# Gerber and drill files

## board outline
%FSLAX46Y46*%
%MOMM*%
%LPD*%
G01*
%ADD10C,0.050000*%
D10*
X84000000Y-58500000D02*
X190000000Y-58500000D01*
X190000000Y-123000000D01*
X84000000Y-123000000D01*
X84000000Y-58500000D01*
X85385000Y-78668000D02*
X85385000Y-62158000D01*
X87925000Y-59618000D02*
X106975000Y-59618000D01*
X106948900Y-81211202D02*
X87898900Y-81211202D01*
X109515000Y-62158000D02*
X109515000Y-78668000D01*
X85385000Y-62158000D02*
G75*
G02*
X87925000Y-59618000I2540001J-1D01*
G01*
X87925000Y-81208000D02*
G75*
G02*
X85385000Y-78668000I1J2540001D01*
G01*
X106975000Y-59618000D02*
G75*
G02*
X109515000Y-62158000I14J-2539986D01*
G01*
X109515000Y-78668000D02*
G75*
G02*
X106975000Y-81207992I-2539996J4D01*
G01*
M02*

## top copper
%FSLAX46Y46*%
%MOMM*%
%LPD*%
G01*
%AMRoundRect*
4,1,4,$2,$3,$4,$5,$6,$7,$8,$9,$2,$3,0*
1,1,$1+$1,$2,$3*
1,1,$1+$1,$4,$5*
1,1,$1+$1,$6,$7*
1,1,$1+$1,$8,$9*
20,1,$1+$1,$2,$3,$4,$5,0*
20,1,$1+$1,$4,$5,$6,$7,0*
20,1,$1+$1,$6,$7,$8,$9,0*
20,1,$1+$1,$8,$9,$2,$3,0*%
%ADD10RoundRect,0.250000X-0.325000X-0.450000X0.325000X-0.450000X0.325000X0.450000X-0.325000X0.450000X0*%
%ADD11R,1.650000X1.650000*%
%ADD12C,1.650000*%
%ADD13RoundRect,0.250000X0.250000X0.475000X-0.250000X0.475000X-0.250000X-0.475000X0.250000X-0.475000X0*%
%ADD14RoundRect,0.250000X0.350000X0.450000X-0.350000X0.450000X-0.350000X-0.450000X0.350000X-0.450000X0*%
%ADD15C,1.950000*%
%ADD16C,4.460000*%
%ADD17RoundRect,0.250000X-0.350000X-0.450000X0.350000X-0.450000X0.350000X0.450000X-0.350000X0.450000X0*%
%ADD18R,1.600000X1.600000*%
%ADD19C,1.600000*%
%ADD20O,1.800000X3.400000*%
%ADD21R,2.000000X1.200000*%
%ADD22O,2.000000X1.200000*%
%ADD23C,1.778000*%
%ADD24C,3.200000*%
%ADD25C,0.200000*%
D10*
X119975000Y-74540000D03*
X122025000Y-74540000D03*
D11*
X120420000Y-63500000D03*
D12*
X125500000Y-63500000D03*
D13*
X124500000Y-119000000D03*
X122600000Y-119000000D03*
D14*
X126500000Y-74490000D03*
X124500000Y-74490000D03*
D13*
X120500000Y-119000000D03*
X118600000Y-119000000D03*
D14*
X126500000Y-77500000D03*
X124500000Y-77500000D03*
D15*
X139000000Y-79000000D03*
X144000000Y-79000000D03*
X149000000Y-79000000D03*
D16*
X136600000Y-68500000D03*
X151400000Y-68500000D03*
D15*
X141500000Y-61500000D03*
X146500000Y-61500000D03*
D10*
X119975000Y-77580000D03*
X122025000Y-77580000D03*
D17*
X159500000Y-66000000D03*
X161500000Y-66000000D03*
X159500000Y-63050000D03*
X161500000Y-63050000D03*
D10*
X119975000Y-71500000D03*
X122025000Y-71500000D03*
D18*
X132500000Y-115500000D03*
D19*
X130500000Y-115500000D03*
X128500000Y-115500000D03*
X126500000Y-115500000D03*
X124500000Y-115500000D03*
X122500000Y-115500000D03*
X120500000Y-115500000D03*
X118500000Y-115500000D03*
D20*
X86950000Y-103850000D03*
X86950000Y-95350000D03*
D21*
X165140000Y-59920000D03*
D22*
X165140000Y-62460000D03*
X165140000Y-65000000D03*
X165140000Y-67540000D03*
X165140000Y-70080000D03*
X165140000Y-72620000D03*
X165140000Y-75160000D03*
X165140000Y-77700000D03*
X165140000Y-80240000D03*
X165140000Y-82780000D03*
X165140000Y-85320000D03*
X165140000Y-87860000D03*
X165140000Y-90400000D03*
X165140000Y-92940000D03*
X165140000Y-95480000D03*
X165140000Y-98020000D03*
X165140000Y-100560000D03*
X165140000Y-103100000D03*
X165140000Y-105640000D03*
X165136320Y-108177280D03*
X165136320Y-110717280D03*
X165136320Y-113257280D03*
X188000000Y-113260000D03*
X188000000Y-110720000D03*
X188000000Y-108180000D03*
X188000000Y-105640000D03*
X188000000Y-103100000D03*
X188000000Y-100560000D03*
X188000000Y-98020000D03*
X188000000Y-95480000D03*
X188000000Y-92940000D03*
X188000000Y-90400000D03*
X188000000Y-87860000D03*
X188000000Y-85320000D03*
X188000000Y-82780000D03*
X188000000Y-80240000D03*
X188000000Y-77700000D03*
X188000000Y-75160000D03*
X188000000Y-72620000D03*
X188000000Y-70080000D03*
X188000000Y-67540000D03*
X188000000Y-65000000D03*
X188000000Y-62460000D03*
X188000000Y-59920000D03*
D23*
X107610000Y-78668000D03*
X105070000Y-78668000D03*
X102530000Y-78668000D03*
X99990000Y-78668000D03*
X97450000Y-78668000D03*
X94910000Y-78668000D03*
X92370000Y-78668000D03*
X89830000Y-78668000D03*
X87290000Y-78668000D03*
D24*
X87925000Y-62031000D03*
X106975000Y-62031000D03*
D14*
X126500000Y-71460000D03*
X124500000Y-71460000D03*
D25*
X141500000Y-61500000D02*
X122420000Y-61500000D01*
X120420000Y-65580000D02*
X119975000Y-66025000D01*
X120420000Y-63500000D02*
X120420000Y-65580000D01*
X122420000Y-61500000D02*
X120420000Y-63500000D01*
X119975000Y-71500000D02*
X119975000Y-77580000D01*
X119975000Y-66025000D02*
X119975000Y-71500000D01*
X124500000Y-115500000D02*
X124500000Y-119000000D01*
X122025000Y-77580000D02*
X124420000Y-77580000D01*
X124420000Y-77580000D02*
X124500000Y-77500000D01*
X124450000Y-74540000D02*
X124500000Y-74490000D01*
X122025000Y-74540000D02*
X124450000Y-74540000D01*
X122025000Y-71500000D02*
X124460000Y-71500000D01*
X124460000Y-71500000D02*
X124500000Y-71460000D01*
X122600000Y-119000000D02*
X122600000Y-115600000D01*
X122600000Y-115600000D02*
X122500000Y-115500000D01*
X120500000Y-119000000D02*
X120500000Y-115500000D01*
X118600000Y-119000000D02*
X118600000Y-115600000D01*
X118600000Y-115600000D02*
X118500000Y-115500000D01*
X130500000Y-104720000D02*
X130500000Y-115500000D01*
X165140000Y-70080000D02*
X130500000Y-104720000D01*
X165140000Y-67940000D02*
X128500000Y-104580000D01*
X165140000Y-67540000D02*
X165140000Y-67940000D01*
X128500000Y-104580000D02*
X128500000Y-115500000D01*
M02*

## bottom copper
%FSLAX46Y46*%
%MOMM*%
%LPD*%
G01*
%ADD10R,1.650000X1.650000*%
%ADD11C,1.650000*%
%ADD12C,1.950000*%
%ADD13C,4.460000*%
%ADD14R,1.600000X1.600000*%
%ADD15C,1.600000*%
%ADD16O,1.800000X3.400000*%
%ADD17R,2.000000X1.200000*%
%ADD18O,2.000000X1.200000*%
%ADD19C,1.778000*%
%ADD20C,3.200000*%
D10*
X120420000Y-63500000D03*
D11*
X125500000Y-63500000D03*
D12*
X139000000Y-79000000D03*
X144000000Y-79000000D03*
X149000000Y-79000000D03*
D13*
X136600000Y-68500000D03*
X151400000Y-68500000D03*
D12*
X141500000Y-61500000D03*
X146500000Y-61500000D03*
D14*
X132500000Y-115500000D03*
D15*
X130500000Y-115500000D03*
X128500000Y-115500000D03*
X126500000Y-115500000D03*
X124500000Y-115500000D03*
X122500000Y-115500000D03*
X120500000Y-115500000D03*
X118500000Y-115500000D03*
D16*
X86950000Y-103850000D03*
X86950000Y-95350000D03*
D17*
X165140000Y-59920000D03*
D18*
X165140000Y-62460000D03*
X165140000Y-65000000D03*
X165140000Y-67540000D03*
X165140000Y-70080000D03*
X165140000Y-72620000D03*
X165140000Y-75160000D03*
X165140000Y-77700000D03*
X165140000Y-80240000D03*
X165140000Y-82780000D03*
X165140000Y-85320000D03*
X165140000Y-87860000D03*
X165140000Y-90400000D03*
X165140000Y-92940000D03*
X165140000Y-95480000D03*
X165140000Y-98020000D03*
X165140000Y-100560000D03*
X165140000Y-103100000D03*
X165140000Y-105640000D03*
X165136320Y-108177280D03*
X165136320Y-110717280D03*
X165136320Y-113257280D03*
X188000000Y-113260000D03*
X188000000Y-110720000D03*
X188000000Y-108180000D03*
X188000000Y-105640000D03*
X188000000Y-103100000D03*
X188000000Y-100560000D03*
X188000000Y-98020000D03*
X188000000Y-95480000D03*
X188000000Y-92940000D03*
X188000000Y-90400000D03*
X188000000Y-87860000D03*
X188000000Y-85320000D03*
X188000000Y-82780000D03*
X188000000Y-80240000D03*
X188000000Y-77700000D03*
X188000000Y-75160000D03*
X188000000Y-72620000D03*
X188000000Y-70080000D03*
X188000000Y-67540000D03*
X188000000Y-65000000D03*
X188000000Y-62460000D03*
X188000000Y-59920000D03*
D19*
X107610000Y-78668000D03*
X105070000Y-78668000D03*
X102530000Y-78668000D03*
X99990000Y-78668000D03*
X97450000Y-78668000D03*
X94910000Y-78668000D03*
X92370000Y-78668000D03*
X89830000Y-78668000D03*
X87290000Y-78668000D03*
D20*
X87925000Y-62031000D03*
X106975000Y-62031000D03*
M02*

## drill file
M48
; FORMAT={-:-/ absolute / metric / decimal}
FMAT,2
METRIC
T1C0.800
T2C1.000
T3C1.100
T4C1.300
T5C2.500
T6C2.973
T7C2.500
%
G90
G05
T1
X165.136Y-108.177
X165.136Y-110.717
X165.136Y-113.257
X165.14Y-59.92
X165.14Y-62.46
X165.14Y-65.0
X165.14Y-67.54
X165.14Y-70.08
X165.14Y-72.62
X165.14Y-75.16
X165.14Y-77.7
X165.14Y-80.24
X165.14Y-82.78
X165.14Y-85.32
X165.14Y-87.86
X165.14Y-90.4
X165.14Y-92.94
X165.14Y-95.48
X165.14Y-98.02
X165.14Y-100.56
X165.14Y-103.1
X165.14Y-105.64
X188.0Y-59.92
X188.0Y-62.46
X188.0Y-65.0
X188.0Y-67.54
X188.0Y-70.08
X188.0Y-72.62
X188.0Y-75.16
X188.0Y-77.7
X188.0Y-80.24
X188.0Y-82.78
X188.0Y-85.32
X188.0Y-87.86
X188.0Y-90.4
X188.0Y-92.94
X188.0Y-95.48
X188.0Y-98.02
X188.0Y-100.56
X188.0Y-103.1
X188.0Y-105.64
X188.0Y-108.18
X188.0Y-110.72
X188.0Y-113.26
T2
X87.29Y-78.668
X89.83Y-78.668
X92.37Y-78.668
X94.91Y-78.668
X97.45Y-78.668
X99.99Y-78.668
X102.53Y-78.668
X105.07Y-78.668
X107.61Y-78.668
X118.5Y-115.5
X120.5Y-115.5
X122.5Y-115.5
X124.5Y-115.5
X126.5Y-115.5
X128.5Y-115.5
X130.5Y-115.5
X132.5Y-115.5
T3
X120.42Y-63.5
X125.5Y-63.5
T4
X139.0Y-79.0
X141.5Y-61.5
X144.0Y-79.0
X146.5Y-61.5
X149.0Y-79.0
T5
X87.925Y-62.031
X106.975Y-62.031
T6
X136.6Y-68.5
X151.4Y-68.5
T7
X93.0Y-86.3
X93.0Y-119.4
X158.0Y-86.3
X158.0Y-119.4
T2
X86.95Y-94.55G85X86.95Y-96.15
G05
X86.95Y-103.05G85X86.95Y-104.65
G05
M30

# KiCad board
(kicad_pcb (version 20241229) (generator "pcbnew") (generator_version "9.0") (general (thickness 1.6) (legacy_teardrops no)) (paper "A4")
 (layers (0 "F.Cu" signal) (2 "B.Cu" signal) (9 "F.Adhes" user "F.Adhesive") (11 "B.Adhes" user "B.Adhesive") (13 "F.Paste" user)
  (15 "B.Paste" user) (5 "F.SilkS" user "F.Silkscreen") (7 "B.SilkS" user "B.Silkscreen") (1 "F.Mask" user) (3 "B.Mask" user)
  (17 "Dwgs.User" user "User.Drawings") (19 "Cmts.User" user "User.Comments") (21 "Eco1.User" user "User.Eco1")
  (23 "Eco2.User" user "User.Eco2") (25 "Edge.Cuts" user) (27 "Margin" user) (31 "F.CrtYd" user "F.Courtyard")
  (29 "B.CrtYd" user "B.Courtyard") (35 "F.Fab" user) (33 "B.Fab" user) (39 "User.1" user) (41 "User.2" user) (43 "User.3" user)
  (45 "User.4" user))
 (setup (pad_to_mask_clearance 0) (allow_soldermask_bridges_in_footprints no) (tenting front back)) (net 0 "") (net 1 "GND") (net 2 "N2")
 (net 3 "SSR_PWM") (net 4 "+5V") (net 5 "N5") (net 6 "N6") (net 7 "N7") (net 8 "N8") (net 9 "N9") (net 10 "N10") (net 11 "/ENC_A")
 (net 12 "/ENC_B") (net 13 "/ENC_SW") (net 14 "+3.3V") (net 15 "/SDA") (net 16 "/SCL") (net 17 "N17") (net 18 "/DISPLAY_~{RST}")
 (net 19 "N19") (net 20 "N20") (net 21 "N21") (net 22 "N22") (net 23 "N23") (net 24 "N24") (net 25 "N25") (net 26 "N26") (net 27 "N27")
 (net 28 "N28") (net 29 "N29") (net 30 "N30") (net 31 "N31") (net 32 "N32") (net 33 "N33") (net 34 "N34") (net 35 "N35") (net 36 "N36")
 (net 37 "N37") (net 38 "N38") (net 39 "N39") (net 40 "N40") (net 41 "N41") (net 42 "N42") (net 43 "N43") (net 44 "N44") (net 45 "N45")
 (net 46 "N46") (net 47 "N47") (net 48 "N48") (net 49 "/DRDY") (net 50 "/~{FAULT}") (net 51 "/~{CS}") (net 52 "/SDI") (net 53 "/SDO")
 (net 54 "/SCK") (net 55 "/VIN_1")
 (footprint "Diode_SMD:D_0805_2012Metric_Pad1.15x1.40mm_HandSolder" (layer "F.Cu") (at 121 74.54)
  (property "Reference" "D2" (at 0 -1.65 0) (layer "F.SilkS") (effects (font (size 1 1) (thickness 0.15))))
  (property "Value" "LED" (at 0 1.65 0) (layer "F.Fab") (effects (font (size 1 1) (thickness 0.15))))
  (pad "1" smd roundrect (at -1.025 0) (size 1.15 1.4) (layers "F.Cu" "F.Mask" "F.Paste") (roundrect_rratio 0.217391) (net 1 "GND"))
  (pad "2" smd roundrect (at 1.025 0) (size 1.15 1.4) (layers "F.Cu" "F.Mask" "F.Paste") (roundrect_rratio 0.217391) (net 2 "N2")))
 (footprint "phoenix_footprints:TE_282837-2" (layer "F.Cu") (at 122.96 63.5)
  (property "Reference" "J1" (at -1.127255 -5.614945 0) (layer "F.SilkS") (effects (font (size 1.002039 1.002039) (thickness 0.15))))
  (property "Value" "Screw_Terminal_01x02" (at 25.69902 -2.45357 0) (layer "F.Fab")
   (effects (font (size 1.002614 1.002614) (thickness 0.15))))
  (pad "1" thru_hole rect (at -2.54 0) (size 1.65 1.65) (drill 1.1) (layers "*.Cu" "*.Mask") (remove_unused_layers no) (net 1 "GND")
   (solder_mask_margin 0.102))
  (pad "2" thru_hole circle (at 2.54 0) (size 1.65 1.65) (drill 1.1) (layers "*.Cu" "*.Mask") (remove_unused_layers no) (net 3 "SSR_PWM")
   (solder_mask_margin 0.102)))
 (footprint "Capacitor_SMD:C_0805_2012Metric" (layer "F.Cu") (at 123.55 119 180)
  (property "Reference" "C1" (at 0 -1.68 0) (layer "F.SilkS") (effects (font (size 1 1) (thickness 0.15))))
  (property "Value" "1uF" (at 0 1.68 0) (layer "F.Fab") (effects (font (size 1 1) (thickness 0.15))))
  (pad "1" smd roundrect (at -0.95 0 180) (size 1 1.45) (layers "F.Cu" "F.Mask" "F.Paste") (roundrect_rratio 0.25) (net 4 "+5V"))
  (pad "2" smd roundrect (at 0.95 0 180) (size 1 1.45) (layers "F.Cu" "F.Mask" "F.Paste") (roundrect_rratio 0.25) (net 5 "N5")))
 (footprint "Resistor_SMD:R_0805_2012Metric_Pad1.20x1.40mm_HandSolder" (layer "F.Cu") (at 125.5 74.49 180)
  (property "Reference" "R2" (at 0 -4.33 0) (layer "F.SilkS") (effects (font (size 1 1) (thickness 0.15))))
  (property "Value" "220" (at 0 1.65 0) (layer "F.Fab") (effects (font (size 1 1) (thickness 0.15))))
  (pad "1" smd roundrect (at -1 0 180) (size 1.2 1.4) (layers "F.Cu" "F.Mask" "F.Paste") (roundrect_rratio 0.208333) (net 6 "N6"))
  (pad "2" smd roundrect (at 1 0 180) (size 1.2 1.4) (layers "F.Cu" "F.Mask" "F.Paste") (roundrect_rratio 0.208333) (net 2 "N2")))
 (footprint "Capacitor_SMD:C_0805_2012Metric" (layer "F.Cu") (at 119.55 119 180)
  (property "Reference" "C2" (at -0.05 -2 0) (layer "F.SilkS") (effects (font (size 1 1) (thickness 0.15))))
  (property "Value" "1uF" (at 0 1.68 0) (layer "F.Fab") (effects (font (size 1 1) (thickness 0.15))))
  (pad "1" smd roundrect (at -0.95 0 180) (size 1 1.45) (layers "F.Cu" "F.Mask" "F.Paste") (roundrect_rratio 0.25) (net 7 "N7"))
  (pad "2" smd roundrect (at 0.95 0 180) (size 1 1.45) (layers "F.Cu" "F.Mask" "F.Paste") (roundrect_rratio 0.25) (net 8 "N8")))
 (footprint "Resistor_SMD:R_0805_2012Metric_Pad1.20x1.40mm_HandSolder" (layer "F.Cu") (at 125.5 77.5 180)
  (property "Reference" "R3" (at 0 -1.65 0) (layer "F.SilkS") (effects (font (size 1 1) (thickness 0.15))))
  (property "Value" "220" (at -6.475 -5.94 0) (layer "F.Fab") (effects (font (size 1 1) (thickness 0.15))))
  (pad "1" smd roundrect (at -1 0 180) (size 1.2 1.4) (layers "F.Cu" "F.Mask" "F.Paste") (roundrect_rratio 0.208333) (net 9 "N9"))
  (pad "2" smd roundrect (at 1 0 180) (size 1.2 1.4) (layers "F.Cu" "F.Mask" "F.Paste") (roundrect_rratio 0.208333) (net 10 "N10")))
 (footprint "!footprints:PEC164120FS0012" (layer "F.Cu") (at 139 79)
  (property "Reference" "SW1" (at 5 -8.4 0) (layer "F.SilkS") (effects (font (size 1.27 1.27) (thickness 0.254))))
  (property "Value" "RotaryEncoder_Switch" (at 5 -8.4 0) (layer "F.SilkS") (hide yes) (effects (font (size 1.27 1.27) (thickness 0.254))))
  (pad "A" thru_hole circle (at 0 0) (size 1.95 1.95) (drill 1.3) (layers "*.Cu" "*.Mask") (remove_unused_layers no) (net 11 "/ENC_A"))
  (pad "B" thru_hole circle (at 5 0) (size 1.95 1.95) (drill 1.3) (layers "*.Cu" "*.Mask") (remove_unused_layers no) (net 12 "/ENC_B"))
  (pad "C" thru_hole circle (at 10 0) (size 1.95 1.95) (drill 1.3) (layers "*.Cu" "*.Mask") (remove_unused_layers no) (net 1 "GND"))
  (pad "MH1" thru_hole circle (at -2.4 -10.5) (size 4.46 4.46) (drill 2.9732) (layers "*.Cu" "*.Mask") (remove_unused_layers no))
  (pad "MH2" thru_hole circle (at 12.4 -10.5) (size 4.46 4.46) (drill 2.9732) (layers "*.Cu" "*.Mask") (remove_unused_layers no))
  (pad "S1" thru_hole circle (at 2.5 -17.5) (size 1.95 1.95) (drill 1.3) (layers "*.Cu" "*.Mask") (remove_unused_layers no) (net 1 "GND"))
  (pad "S2" thru_hole circle (at 7.5 -17.5) (size 1.95 1.95) (drill 1.3) (layers "*.Cu" "*.Mask") (remove_unused_layers no)
   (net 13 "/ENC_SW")))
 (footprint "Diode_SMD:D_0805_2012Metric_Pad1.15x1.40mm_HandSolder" (layer "F.Cu") (at 121 77.58)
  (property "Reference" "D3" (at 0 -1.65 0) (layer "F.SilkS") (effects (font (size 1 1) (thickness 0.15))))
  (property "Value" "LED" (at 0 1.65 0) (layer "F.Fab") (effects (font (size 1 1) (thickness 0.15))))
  (pad "1" smd roundrect (at -1.025 0) (size 1.15 1.4) (layers "F.Cu" "F.Mask" "F.Paste") (roundrect_rratio 0.217391) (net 1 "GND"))
  (pad "2" smd roundrect (at 1.025 0) (size 1.15 1.4) (layers "F.Cu" "F.Mask" "F.Paste") (roundrect_rratio 0.217391) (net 10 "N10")))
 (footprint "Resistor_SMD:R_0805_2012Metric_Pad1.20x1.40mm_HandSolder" (layer "F.Cu") (at 160.5 66)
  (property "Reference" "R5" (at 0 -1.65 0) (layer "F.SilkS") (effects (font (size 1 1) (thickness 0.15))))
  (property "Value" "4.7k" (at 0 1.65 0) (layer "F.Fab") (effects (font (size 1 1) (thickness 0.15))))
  (pad "1" smd roundrect (at -1 0) (size 1.2 1.4) (layers "F.Cu" "F.Mask" "F.Paste") (roundrect_rratio 0.208333) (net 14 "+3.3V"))
  (pad "2" smd roundrect (at 1 0) (size 1.2 1.4) (layers "F.Cu" "F.Mask" "F.Paste") (roundrect_rratio 0.208333) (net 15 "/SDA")))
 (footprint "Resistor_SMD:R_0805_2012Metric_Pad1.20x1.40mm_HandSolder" (layer "F.Cu") (at 160.5 63.05)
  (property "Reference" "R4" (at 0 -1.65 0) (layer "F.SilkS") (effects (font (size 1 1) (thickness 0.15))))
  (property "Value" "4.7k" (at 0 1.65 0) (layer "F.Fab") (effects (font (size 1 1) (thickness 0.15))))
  (pad "1" smd roundrect (at -1 0) (size 1.2 1.4) (layers "F.Cu" "F.Mask" "F.Paste") (roundrect_rratio 0.208333) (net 14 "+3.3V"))
  (pad "2" smd roundrect (at 1 0) (size 1.2 1.4) (layers "F.Cu" "F.Mask" "F.Paste") (roundrect_rratio 0.208333) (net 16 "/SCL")))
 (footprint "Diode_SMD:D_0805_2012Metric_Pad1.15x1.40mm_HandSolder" (layer "F.Cu") (at 121 71.5)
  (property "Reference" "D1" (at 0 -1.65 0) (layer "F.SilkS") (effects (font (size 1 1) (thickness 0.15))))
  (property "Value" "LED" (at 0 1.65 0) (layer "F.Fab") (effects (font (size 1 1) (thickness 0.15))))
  (pad "1" smd roundrect (at -1.025 0) (size 1.15 1.4) (layers "F.Cu" "F.Mask" "F.Paste") (roundrect_rratio 0.217391) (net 1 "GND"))
  (pad "2" smd roundrect (at 1.025 0) (size 1.15 1.4) (layers "F.Cu" "F.Mask" "F.Paste") (roundrect_rratio 0.217391) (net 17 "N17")))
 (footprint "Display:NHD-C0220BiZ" (layer "F.Cu") (at 125.5 99.6)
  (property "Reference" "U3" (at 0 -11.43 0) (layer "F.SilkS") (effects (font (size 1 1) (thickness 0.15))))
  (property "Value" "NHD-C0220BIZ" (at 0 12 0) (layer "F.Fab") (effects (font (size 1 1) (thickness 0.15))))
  (pad "" np_thru_hole circle (at -32.5 -13.3) (size 2.5 2.5) (drill 2.5) (layers "*.Cu" "*.Mask"))
  (pad "" np_thru_hole circle (at -32.5 19.8) (size 2.5 2.5) (drill 2.5) (layers "*.Cu" "*.Mask"))
  (pad "" np_thru_hole circle (at 32.5 -13.3) (size 2.5 2.5) (drill 2.5) (layers "*.Cu" "*.Mask"))
  (pad "" np_thru_hole circle (at 32.5 19.8) (size 2.5 2.5) (drill 2.5) (layers "*.Cu" "*.Mask"))
  (pad "1" thru_hole rect (at 7 15.9) (size 1.6 1.6) (drill 1) (layers "*.Cu" "*.Mask") (remove_unused_layers no) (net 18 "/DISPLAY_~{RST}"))
  (pad "2" thru_hole circle (at 5 15.9) (size 1.6 1.6) (drill 1) (layers "*.Cu" "*.Mask") (remove_unused_layers no) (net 16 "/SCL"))
  (pad "3" thru_hole circle (at 3 15.9) (size 1.6 1.6) (drill 1) (layers "*.Cu" "*.Mask") (remove_unused_layers no) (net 15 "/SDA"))
  (pad "4" thru_hole circle (at 1 15.9) (size 1.6 1.6) (drill 1) (layers "*.Cu" "*.Mask") (remove_unused_layers no) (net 1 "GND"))
  (pad "5" thru_hole circle (at -1 15.9) (size 1.6 1.6) (drill 1) (layers "*.Cu" "*.Mask") (remove_unused_layers no) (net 4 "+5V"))
  (pad "6" thru_hole circle (at -3 15.9) (size 1.6 1.6) (drill 1) (layers "*.Cu" "*.Mask") (remove_unused_layers no) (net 5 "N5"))
  (pad "7" thru_hole circle (at -5 15.9) (size 1.6 1.6) (drill 1) (layers "*.Cu" "*.Mask") (remove_unused_layers no) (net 7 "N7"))
  (pad "8" thru_hole circle (at -7 15.9) (size 1.6 1.6) (drill 1) (layers "*.Cu" "*.Mask") (remove_unused_layers no) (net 8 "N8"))
  (pad "9" thru_hole oval (at -38.55 4.25) (size 1.8 3.4) (drill oval 1 2.6) (layers "*.Cu" "*.Mask") (remove_unused_layers no)
   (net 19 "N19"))
  (pad "10" thru_hole oval (at -38.55 -4.25) (size 1.8 3.4) (drill oval 1 2.6) (layers "*.Cu" "*.Mask") (remove_unused_layers no)
   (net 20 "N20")))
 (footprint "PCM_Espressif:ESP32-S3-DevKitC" (layer "F.Cu") (at 165.14 59.92)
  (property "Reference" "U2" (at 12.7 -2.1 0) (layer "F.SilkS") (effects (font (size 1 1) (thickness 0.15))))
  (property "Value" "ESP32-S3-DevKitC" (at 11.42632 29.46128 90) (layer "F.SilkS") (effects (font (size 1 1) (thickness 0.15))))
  (pad "1" thru_hole rect (at 0 0 270) (size 1.2 2) (drill 0.8) (layers "*.Cu" "*.Mask") (remove_unused_layers no) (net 14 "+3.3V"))
  (pad "2" thru_hole oval (at 0 2.54 270) (size 1.2 2) (drill 0.8) (layers "*.Cu" "*.Mask") (remove_unused_layers no) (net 14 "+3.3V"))
  (pad "3" thru_hole oval (at 0 5.08 270) (size 1.2 2) (drill 0.8) (layers "*.Cu" "*.Mask") (remove_unused_layers no) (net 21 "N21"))
  (pad "4" thru_hole oval (at 0 7.62 270) (size 1.2 2) (drill 0.8) (layers "*.Cu" "*.Mask") (remove_unused_layers no) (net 15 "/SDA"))
  (pad "5" thru_hole oval (at 0 10.16 270) (size 1.2 2) (drill 0.8) (layers "*.Cu" "*.Mask") (remove_unused_layers no) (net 16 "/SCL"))
  (pad "6" thru_hole oval (at 0 12.7 270) (size 1.2 2) (drill 0.8) (layers "*.Cu" "*.Mask") (remove_unused_layers no) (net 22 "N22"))
  (pad "7" thru_hole oval (at 0 15.24 270) (size 1.2 2) (drill 0.8) (layers "*.Cu" "*.Mask") (remove_unused_layers no) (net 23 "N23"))
  (pad "8" thru_hole oval (at 0 17.78 270) (size 1.2 2) (drill 0.8) (layers "*.Cu" "*.Mask") (remove_unused_layers no) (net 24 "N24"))
  (pad "9" thru_hole oval (at 0 20.32 270) (size 1.2 2) (drill 0.8) (layers "*.Cu" "*.Mask") (remove_unused_layers no) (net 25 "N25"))
  (pad "10" thru_hole oval (at 0 22.86 270) (size 1.2 2) (drill 0.8) (layers "*.Cu" "*.Mask") (remove_unused_layers no) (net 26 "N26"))
  (pad "11" thru_hole oval (at 0 25.4 270) (size 1.2 2) (drill 0.8) (layers "*.Cu" "*.Mask") (remove_unused_layers no) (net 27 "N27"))
  (pad "12" thru_hole oval (at 0 27.94 270) (size 1.2 2) (drill 0.8) (layers "*.Cu" "*.Mask") (remove_unused_layers no) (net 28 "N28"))
  (pad "13" thru_hole oval (at 0 30.48 270) (size 1.2 2) (drill 0.8) (layers "*.Cu" "*.Mask") (remove_unused_layers no) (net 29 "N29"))
  (pad "14" thru_hole oval (at 0 33.02 270) (size 1.2 2) (drill 0.8) (layers "*.Cu" "*.Mask") (remove_unused_layers no) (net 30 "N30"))
  (pad "15" thru_hole oval (at 0 35.56 270) (size 1.2 2) (drill 0.8) (layers "*.Cu" "*.Mask") (remove_unused_layers no) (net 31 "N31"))
  (pad "16" thru_hole oval (at 0 38.1 270) (size 1.2 2) (drill 0.8) (layers "*.Cu" "*.Mask") (remove_unused_layers no) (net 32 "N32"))
  (pad "17" thru_hole oval (at 0 40.64 270) (size 1.2 2) (drill 0.8) (layers "*.Cu" "*.Mask") (remove_unused_layers no) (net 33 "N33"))
  (pad "18" thru_hole oval (at 0 43.18 270) (size 1.2 2) (drill 0.8) (layers "*.Cu" "*.Mask") (remove_unused_layers no) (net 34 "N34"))
  (pad "19" thru_hole oval (at 0 45.72 270) (size 1.2 2) (drill 0.8) (layers "*.Cu" "*.Mask") (remove_unused_layers no) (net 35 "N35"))
  (pad "20" thru_hole oval (at -0.00368 48.25728 270) (size 1.2 2) (drill 0.8) (layers "*.Cu" "*.Mask") (remove_unused_layers no)
   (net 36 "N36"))
  (pad "21" thru_hole oval (at -0.00368 50.79728 270) (size 1.2 2) (drill 0.8) (layers "*.Cu" "*.Mask") (remove_unused_layers no)
   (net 4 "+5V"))
  (pad "22" thru_hole oval (at -0.00368 53.33728 270) (size 1.2 2) (drill 0.8) (layers "*.Cu" "*.Mask") (remove_unused_layers no)
   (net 1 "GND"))
  (pad "23" thru_hole oval (at 22.86 53.34 270) (size 1.2 2) (drill 0.8) (layers "*.Cu" "*.Mask") (remove_unused_layers no) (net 1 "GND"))
  (pad "24" thru_hole oval (at 22.86 50.8 270) (size 1.2 2) (drill 0.8) (layers "*.Cu" "*.Mask") (remove_unused_layers no) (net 1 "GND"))
  (pad "25" thru_hole oval (at 22.86 48.26 270) (size 1.2 2) (drill 0.8) (layers "*.Cu" "*.Mask") (remove_unused_layers no) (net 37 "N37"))
  (pad "26" thru_hole oval (at 22.86 45.72 270) (size 1.2 2) (drill 0.8) (layers "*.Cu" "*.Mask") (remove_unused_layers no) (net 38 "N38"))
  (pad "27" thru_hole oval (at 22.86 43.18 270) (size 1.2 2) (drill 0.8) (layers "*.Cu" "*.Mask") (remove_unused_layers no)
   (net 3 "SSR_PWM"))
  (pad "28" thru_hole oval (at 22.86 40.64 270) (size 1.2 2) (drill 0.8) (layers "*.Cu" "*.Mask") (remove_unused_layers no) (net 6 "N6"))
  (pad "29" thru_hole oval (at 22.86 38.1 270) (size 1.2 2) (drill 0.8) (layers "*.Cu" "*.Mask") (remove_unused_layers no) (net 9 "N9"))
  (pad "30" thru_hole oval (at 22.86 35.56 270) (size 1.2 2) (drill 0.8) (layers "*.Cu" "*.Mask") (remove_unused_layers no) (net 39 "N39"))
  (pad "31" thru_hole oval (at 22.86 33.02 270) (size 1.2 2) (drill 0.8) (layers "*.Cu" "*.Mask") (remove_unused_layers no) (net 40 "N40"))
  (pad "32" thru_hole oval (at 22.86 30.48 270) (size 1.2 2) (drill 0.8) (layers "*.Cu" "*.Mask") (remove_unused_layers no)
   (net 18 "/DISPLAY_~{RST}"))
  (pad "33" thru_hole oval (at 22.86 27.94 270) (size 1.2 2) (drill 0.8) (layers "*.Cu" "*.Mask") (remove_unused_layers no)
   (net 11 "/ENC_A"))
  (pad "34" thru_hole oval (at 22.86 25.4 270) (size 1.2 2) (drill 0.8) (layers "*.Cu" "*.Mask") (remove_unused_layers no) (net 12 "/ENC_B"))
  (pad "35" thru_hole oval (at 22.86 22.86 270) (size 1.2 2) (drill 0.8) (layers "*.Cu" "*.Mask") (remove_unused_layers no)
   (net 13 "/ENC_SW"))
  (pad "36" thru_hole oval (at 22.86 20.32 270) (size 1.2 2) (drill 0.8) (layers "*.Cu" "*.Mask") (remove_unused_layers no) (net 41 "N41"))
  (pad "37" thru_hole oval (at 22.86 17.78 270) (size 1.2 2) (drill 0.8) (layers "*.Cu" "*.Mask") (remove_unused_layers no) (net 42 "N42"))
  (pad "38" thru_hole oval (at 22.86 15.24 270) (size 1.2 2) (drill 0.8) (layers "*.Cu" "*.Mask") (remove_unused_layers no) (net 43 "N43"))
  (pad "39" thru_hole oval (at 22.86 12.7 270) (size 1.2 2) (drill 0.8) (layers "*.Cu" "*.Mask") (remove_unused_layers no) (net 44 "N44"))
  (pad "40" thru_hole oval (at 22.86 10.16 270) (size 1.2 2) (drill 0.8) (layers "*.Cu" "*.Mask") (remove_unused_layers no) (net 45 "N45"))
  (pad "41" thru_hole oval (at 22.86 7.62 270) (size 1.2 2) (drill 0.8) (layers "*.Cu" "*.Mask") (remove_unused_layers no) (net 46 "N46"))
  (pad "42" thru_hole oval (at 22.86 5.08 270) (size 1.2 2) (drill 0.8) (layers "*.Cu" "*.Mask") (remove_unused_layers no) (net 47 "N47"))
  (pad "43" thru_hole oval (at 22.86 2.54 270) (size 1.2 2) (drill 0.8) (layers "*.Cu" "*.Mask") (remove_unused_layers no) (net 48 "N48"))
  (pad "44" thru_hole oval (at 22.86 0 270) (size 1.2 2) (drill 0.8) (layers "*.Cu" "*.Mask") (remove_unused_layers no) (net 1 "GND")))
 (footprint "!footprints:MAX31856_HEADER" (layer "F.Cu") (at 87.936314 62.019686)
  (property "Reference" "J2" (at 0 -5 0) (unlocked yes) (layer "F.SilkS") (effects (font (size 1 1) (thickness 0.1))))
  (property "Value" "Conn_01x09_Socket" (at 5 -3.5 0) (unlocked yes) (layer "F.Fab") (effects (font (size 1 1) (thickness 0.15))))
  (fp_line (start -2.551314 16.648314) (end -2.551314 0.138314) (stroke (width 0.05) (type solid)) (layer "Edge.Cuts"))
  (fp_line (start -0.011314 -2.401686) (end 19.038686 -2.401686) (stroke (width 0.05) (type solid)) (layer "Edge.Cuts"))
  (fp_line (start 19.012586 19.191516) (end -0.037414 19.191516) (stroke (width 0.05) (type solid)) (layer "Edge.Cuts"))
  (fp_line (start 21.578686 0.138314) (end 21.578686 16.648314) (stroke (width 0.05) (type solid)) (layer "Edge.Cuts"))
  (fp_arc (start -2.551314 0.138314) (mid -1.807365 -1.657737) (end -0.011314 -2.401686) (stroke (width 0.05) (type solid))
   (layer "Edge.Cuts"))
  (fp_arc (start -0.011314 19.188314) (mid -1.807365 18.444365) (end -2.551314 16.648314) (stroke (width 0.05) (type solid))
   (layer "Edge.Cuts"))
  (fp_arc (start 19.038686 -2.401686) (mid 20.834737 -1.657737) (end 21.578686 0.138314) (stroke (width 0.05) (type solid))
   (layer "Edge.Cuts"))
  (fp_arc (start 21.578686 16.648314) (mid 20.834737 18.444365) (end 19.038686 19.188314) (stroke (width 0.05) (type solid))
   (layer "Edge.Cuts"))
  (pad "1" thru_hole circle (at 19.673686 16.648314 270) (size 1.778 1.778) (drill 1) (layers "*.Cu" "*.Mask") (remove_unused_layers no)
   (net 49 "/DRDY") (solder_mask_margin 0.0508) (thermal_bridge_angle 0))
  (pad "2" thru_hole circle (at 17.133686 16.648314 270) (size 1.778 1.778) (drill 1) (layers "*.Cu" "*.Mask") (remove_unused_layers no)
   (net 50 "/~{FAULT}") (solder_mask_margin 0.0508) (thermal_bridge_angle 0))
  (pad "3" thru_hole circle (at 14.593686 16.648314 270) (size 1.778 1.778) (drill 1) (layers "*.Cu" "*.Mask") (remove_unused_layers no)
   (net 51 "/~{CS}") (solder_mask_margin 0.0508) (thermal_bridge_angle 0))
  (pad "4" thru_hole circle (at 12.053686 16.648314 270) (size 1.778 1.778) (drill 1) (layers "*.Cu" "*.Mask") (remove_unused_layers no)
   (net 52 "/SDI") (solder_mask_margin 0.0508) (thermal_bridge_angle 0))
  (pad "5" thru_hole circle (at 9.513686 16.648314 270) (size 1.778 1.778) (drill 1) (layers "*.Cu" "*.Mask") (remove_unused_layers no)
   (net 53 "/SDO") (solder_mask_margin 0.0508) (thermal_bridge_angle 0))
  (pad "6" thru_hole circle (at 6.973686 16.648314 270) (size 1.778 1.778) (drill 1) (layers "*.Cu" "*.Mask") (remove_unused_layers no)
   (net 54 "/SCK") (solder_mask_margin 0.0508) (thermal_bridge_angle 0))
  (pad "7" thru_hole circle (at 4.433686 16.648314 270) (size 1.778 1.778) (drill 1) (layers "*.Cu" "*.Mask") (remove_unused_layers no)
   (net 1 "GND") (solder_mask_margin 0.0508) (thermal_bridge_angle 0))
  (pad "8" thru_hole circle (at 1.893686 16.648314 270) (size 1.778 1.778) (drill 1) (layers "*.Cu" "*.Mask") (remove_unused_layers no)
   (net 14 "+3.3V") (solder_mask_margin 0.0508) (thermal_bridge_angle 0))
  (pad "9" thru_hole circle (at -0.646314 16.648314 270) (size 1.778 1.778) (drill 1) (layers "*.Cu" "*.Mask") (remove_unused_layers no)
   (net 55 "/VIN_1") (solder_mask_margin 0.0508) (thermal_bridge_angle 0))
  (pad "P$1" thru_hole circle (at -0.011314 0.011314) (size 3.2 3.2) (drill 2.5) (layers "*.Cu" "*.Mask") (remove_unused_layers no)
   (solder_mask_margin 0.0508) (thermal_bridge_angle 0))
  (pad "P$1" thru_hole circle (at 19.038686 0.011314) (size 3.2 3.2) (drill 2.5) (layers "*.Cu" "*.Mask") (remove_unused_layers no)
   (solder_mask_margin 0.0508) (thermal_bridge_angle 0))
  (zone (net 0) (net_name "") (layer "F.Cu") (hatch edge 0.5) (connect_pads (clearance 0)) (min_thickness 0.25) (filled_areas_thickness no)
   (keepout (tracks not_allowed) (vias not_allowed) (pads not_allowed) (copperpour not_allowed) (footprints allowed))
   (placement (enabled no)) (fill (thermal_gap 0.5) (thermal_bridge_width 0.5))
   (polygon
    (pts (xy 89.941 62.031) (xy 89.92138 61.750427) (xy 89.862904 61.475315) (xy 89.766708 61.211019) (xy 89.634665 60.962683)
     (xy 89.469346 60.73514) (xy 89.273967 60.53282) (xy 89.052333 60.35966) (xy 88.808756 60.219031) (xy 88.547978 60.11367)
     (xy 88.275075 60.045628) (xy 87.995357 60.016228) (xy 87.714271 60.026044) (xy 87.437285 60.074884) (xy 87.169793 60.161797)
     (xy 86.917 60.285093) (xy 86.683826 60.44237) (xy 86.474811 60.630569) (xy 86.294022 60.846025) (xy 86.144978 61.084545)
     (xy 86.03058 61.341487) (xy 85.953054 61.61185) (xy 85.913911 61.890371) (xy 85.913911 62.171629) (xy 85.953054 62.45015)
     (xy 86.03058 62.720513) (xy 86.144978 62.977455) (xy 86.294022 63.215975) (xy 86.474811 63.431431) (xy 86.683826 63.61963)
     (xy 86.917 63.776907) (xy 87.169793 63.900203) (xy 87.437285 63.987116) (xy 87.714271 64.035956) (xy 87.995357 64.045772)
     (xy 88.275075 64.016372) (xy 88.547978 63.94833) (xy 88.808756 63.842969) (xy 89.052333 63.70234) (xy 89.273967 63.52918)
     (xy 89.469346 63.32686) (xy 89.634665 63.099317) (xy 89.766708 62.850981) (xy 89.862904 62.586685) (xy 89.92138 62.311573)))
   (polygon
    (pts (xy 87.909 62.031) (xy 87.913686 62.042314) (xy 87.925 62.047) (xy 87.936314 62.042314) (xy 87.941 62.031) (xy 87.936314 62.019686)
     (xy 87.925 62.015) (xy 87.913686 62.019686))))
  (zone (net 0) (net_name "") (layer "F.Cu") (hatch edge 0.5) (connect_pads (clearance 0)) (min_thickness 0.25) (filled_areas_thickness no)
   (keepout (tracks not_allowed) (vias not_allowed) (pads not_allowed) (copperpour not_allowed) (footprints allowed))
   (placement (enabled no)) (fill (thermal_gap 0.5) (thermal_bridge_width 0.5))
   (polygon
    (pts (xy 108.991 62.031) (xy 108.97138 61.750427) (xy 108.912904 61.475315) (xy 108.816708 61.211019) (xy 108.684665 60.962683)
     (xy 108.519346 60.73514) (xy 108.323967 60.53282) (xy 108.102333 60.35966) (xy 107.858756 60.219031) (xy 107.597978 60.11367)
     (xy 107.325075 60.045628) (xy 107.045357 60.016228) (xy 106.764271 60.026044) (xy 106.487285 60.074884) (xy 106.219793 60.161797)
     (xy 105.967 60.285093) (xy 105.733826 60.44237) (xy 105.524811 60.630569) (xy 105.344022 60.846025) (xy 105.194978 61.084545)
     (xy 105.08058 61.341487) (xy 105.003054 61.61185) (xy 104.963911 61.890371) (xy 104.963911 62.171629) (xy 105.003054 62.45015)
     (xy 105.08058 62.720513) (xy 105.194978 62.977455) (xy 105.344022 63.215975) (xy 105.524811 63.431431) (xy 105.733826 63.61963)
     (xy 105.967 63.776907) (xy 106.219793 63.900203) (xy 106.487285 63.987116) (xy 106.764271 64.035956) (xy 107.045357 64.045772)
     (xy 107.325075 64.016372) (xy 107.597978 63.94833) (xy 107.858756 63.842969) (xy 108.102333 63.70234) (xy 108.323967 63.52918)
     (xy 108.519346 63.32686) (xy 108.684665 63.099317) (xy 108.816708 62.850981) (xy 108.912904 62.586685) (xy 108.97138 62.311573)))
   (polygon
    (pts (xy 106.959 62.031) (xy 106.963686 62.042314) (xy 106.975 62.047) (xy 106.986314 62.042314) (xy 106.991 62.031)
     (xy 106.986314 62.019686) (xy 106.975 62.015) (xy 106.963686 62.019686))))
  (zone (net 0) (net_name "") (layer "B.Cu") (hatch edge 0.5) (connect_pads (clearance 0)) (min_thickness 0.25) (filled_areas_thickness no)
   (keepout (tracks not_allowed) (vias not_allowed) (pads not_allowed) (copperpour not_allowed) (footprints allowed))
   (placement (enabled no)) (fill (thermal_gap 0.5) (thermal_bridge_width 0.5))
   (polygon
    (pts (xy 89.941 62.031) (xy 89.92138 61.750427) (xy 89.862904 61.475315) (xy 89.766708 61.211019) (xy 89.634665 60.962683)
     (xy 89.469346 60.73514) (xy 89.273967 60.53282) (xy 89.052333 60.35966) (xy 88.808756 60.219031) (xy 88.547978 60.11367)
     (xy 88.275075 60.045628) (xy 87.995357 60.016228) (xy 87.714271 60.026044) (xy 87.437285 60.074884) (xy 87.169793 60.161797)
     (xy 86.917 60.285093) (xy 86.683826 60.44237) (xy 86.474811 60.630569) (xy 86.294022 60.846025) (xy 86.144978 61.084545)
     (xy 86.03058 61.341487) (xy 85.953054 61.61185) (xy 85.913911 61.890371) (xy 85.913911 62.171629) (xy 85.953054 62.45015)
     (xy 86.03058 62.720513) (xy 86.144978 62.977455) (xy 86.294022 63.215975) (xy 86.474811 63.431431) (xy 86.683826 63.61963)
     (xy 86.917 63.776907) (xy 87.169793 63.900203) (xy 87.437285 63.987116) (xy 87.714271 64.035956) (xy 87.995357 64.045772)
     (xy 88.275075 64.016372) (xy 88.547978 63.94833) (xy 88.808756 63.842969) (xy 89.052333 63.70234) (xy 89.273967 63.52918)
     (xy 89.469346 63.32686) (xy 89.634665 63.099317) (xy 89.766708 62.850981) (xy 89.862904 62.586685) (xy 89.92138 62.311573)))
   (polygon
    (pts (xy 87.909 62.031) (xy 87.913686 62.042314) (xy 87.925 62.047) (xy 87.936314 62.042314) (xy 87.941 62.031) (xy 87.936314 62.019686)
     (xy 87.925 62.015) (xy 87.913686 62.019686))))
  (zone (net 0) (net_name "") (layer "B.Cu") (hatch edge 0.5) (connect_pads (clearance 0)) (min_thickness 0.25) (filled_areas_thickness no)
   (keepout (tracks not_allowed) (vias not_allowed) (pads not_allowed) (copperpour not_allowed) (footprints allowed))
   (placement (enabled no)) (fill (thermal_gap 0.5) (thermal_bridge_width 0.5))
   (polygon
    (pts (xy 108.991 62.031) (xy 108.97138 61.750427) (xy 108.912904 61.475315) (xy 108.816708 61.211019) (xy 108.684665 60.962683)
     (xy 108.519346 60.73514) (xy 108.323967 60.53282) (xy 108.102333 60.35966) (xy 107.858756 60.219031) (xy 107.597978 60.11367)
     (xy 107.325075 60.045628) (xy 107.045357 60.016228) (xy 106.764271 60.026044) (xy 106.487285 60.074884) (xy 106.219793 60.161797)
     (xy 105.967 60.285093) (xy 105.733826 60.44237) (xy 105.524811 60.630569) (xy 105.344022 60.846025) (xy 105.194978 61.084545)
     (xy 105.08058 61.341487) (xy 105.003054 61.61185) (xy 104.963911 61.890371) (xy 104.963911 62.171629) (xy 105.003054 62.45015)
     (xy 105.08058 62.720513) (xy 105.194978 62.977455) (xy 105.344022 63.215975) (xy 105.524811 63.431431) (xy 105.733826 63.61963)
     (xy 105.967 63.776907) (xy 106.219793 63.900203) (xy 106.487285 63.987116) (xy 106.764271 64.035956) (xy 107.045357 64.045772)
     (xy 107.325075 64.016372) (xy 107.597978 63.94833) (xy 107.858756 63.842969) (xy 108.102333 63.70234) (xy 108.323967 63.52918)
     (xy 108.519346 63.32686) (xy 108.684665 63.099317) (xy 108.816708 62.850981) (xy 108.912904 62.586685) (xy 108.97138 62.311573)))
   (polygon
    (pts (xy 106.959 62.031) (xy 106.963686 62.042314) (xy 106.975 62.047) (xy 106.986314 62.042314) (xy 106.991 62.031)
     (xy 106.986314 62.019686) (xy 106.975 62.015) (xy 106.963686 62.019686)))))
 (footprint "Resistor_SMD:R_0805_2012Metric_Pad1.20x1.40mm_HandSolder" (layer "F.Cu") (at 125.5 71.46 180)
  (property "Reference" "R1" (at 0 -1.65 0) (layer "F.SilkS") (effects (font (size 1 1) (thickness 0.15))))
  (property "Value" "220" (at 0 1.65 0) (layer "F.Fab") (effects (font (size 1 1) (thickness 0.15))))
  (pad "1" smd roundrect (at -1 0 180) (size 1.2 1.4) (layers "F.Cu" "F.Mask" "F.Paste") (roundrect_rratio 0.208333) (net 30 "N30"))
  (pad "2" smd roundrect (at 1 0 180) (size 1.2 1.4) (layers "F.Cu" "F.Mask" "F.Paste") (roundrect_rratio 0.208333) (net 17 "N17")))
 (gr_rect (start 84 58.5) (end 190 123) (stroke (width 0.05) (type default)) (fill no) (layer "Edge.Cuts"))
 (segment (start 141.5 61.5) (end 122.42 61.5) (width 0.2) (layer "F.Cu") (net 1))
 (segment (start 120.42 65.58) (end 119.975 66.025) (width 0.2) (layer "F.Cu") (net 1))
 (segment (start 120.42 63.5) (end 120.42 65.58) (width 0.2) (layer "F.Cu") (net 1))
 (segment (start 122.42 61.5) (end 120.42 63.5) (width 0.2) (layer "F.Cu") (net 1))
 (segment (start 119.975 71.5) (end 119.975 77.58) (width 0.2) (layer "F.Cu") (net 1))
 (segment (start 119.975 66.025) (end 119.975 71.5) (width 0.2) (layer "F.Cu") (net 1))
 (segment (start 124.5 115.5) (end 124.5 119) (width 0.2) (layer "F.Cu") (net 4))
 (segment (start 122.025 77.58) (end 124.42 77.58) (width 0.2) (layer "F.Cu") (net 10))
 (segment (start 124.42 77.58) (end 124.5 77.5) (width 0.2) (layer "F.Cu") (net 10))
 (segment (start 124.45 74.54) (end 124.5 74.49) (width 0.2) (layer "F.Cu") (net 2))
 (segment (start 122.025 74.54) (end 124.45 74.54) (width 0.2) (layer "F.Cu") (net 2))
 (segment (start 122.025 71.5) (end 124.46 71.5) (width 0.2) (layer "F.Cu") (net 17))
 (segment (start 124.46 71.5) (end 124.5 71.46) (width 0.2) (layer "F.Cu") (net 17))
 (segment (start 122.6 119) (end 122.6 115.6) (width 0.2) (layer "F.Cu") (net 5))
 (segment (start 122.6 115.6) (end 122.5 115.5) (width 0.2) (layer "F.Cu") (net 5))
 (segment (start 120.5 119) (end 120.5 115.5) (width 0.2) (layer "F.Cu") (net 7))
 (segment (start 118.6 119) (end 118.6 115.6) (width 0.2) (layer "F.Cu") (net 8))
 (segment (start 118.6 115.6) (end 118.5 115.5) (width 0.2) (layer "F.Cu") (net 8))
 (segment (start 130.5 104.72) (end 130.5 115.5) (width 0.2) (layer "F.Cu") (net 16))
 (segment (start 165.14 70.08) (end 130.5 104.72) (width 0.2) (layer "F.Cu") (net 16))
 (segment (start 165.14 67.94) (end 128.5 104.58) (width 0.2) (layer "F.Cu") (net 15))
 (segment (start 165.14 67.54) (end 165.14 67.94) (width 0.2) (layer "F.Cu") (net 15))
 (segment (start 128.5 104.58) (end 128.5 115.5) (width 0.2) (layer "F.Cu") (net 15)))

